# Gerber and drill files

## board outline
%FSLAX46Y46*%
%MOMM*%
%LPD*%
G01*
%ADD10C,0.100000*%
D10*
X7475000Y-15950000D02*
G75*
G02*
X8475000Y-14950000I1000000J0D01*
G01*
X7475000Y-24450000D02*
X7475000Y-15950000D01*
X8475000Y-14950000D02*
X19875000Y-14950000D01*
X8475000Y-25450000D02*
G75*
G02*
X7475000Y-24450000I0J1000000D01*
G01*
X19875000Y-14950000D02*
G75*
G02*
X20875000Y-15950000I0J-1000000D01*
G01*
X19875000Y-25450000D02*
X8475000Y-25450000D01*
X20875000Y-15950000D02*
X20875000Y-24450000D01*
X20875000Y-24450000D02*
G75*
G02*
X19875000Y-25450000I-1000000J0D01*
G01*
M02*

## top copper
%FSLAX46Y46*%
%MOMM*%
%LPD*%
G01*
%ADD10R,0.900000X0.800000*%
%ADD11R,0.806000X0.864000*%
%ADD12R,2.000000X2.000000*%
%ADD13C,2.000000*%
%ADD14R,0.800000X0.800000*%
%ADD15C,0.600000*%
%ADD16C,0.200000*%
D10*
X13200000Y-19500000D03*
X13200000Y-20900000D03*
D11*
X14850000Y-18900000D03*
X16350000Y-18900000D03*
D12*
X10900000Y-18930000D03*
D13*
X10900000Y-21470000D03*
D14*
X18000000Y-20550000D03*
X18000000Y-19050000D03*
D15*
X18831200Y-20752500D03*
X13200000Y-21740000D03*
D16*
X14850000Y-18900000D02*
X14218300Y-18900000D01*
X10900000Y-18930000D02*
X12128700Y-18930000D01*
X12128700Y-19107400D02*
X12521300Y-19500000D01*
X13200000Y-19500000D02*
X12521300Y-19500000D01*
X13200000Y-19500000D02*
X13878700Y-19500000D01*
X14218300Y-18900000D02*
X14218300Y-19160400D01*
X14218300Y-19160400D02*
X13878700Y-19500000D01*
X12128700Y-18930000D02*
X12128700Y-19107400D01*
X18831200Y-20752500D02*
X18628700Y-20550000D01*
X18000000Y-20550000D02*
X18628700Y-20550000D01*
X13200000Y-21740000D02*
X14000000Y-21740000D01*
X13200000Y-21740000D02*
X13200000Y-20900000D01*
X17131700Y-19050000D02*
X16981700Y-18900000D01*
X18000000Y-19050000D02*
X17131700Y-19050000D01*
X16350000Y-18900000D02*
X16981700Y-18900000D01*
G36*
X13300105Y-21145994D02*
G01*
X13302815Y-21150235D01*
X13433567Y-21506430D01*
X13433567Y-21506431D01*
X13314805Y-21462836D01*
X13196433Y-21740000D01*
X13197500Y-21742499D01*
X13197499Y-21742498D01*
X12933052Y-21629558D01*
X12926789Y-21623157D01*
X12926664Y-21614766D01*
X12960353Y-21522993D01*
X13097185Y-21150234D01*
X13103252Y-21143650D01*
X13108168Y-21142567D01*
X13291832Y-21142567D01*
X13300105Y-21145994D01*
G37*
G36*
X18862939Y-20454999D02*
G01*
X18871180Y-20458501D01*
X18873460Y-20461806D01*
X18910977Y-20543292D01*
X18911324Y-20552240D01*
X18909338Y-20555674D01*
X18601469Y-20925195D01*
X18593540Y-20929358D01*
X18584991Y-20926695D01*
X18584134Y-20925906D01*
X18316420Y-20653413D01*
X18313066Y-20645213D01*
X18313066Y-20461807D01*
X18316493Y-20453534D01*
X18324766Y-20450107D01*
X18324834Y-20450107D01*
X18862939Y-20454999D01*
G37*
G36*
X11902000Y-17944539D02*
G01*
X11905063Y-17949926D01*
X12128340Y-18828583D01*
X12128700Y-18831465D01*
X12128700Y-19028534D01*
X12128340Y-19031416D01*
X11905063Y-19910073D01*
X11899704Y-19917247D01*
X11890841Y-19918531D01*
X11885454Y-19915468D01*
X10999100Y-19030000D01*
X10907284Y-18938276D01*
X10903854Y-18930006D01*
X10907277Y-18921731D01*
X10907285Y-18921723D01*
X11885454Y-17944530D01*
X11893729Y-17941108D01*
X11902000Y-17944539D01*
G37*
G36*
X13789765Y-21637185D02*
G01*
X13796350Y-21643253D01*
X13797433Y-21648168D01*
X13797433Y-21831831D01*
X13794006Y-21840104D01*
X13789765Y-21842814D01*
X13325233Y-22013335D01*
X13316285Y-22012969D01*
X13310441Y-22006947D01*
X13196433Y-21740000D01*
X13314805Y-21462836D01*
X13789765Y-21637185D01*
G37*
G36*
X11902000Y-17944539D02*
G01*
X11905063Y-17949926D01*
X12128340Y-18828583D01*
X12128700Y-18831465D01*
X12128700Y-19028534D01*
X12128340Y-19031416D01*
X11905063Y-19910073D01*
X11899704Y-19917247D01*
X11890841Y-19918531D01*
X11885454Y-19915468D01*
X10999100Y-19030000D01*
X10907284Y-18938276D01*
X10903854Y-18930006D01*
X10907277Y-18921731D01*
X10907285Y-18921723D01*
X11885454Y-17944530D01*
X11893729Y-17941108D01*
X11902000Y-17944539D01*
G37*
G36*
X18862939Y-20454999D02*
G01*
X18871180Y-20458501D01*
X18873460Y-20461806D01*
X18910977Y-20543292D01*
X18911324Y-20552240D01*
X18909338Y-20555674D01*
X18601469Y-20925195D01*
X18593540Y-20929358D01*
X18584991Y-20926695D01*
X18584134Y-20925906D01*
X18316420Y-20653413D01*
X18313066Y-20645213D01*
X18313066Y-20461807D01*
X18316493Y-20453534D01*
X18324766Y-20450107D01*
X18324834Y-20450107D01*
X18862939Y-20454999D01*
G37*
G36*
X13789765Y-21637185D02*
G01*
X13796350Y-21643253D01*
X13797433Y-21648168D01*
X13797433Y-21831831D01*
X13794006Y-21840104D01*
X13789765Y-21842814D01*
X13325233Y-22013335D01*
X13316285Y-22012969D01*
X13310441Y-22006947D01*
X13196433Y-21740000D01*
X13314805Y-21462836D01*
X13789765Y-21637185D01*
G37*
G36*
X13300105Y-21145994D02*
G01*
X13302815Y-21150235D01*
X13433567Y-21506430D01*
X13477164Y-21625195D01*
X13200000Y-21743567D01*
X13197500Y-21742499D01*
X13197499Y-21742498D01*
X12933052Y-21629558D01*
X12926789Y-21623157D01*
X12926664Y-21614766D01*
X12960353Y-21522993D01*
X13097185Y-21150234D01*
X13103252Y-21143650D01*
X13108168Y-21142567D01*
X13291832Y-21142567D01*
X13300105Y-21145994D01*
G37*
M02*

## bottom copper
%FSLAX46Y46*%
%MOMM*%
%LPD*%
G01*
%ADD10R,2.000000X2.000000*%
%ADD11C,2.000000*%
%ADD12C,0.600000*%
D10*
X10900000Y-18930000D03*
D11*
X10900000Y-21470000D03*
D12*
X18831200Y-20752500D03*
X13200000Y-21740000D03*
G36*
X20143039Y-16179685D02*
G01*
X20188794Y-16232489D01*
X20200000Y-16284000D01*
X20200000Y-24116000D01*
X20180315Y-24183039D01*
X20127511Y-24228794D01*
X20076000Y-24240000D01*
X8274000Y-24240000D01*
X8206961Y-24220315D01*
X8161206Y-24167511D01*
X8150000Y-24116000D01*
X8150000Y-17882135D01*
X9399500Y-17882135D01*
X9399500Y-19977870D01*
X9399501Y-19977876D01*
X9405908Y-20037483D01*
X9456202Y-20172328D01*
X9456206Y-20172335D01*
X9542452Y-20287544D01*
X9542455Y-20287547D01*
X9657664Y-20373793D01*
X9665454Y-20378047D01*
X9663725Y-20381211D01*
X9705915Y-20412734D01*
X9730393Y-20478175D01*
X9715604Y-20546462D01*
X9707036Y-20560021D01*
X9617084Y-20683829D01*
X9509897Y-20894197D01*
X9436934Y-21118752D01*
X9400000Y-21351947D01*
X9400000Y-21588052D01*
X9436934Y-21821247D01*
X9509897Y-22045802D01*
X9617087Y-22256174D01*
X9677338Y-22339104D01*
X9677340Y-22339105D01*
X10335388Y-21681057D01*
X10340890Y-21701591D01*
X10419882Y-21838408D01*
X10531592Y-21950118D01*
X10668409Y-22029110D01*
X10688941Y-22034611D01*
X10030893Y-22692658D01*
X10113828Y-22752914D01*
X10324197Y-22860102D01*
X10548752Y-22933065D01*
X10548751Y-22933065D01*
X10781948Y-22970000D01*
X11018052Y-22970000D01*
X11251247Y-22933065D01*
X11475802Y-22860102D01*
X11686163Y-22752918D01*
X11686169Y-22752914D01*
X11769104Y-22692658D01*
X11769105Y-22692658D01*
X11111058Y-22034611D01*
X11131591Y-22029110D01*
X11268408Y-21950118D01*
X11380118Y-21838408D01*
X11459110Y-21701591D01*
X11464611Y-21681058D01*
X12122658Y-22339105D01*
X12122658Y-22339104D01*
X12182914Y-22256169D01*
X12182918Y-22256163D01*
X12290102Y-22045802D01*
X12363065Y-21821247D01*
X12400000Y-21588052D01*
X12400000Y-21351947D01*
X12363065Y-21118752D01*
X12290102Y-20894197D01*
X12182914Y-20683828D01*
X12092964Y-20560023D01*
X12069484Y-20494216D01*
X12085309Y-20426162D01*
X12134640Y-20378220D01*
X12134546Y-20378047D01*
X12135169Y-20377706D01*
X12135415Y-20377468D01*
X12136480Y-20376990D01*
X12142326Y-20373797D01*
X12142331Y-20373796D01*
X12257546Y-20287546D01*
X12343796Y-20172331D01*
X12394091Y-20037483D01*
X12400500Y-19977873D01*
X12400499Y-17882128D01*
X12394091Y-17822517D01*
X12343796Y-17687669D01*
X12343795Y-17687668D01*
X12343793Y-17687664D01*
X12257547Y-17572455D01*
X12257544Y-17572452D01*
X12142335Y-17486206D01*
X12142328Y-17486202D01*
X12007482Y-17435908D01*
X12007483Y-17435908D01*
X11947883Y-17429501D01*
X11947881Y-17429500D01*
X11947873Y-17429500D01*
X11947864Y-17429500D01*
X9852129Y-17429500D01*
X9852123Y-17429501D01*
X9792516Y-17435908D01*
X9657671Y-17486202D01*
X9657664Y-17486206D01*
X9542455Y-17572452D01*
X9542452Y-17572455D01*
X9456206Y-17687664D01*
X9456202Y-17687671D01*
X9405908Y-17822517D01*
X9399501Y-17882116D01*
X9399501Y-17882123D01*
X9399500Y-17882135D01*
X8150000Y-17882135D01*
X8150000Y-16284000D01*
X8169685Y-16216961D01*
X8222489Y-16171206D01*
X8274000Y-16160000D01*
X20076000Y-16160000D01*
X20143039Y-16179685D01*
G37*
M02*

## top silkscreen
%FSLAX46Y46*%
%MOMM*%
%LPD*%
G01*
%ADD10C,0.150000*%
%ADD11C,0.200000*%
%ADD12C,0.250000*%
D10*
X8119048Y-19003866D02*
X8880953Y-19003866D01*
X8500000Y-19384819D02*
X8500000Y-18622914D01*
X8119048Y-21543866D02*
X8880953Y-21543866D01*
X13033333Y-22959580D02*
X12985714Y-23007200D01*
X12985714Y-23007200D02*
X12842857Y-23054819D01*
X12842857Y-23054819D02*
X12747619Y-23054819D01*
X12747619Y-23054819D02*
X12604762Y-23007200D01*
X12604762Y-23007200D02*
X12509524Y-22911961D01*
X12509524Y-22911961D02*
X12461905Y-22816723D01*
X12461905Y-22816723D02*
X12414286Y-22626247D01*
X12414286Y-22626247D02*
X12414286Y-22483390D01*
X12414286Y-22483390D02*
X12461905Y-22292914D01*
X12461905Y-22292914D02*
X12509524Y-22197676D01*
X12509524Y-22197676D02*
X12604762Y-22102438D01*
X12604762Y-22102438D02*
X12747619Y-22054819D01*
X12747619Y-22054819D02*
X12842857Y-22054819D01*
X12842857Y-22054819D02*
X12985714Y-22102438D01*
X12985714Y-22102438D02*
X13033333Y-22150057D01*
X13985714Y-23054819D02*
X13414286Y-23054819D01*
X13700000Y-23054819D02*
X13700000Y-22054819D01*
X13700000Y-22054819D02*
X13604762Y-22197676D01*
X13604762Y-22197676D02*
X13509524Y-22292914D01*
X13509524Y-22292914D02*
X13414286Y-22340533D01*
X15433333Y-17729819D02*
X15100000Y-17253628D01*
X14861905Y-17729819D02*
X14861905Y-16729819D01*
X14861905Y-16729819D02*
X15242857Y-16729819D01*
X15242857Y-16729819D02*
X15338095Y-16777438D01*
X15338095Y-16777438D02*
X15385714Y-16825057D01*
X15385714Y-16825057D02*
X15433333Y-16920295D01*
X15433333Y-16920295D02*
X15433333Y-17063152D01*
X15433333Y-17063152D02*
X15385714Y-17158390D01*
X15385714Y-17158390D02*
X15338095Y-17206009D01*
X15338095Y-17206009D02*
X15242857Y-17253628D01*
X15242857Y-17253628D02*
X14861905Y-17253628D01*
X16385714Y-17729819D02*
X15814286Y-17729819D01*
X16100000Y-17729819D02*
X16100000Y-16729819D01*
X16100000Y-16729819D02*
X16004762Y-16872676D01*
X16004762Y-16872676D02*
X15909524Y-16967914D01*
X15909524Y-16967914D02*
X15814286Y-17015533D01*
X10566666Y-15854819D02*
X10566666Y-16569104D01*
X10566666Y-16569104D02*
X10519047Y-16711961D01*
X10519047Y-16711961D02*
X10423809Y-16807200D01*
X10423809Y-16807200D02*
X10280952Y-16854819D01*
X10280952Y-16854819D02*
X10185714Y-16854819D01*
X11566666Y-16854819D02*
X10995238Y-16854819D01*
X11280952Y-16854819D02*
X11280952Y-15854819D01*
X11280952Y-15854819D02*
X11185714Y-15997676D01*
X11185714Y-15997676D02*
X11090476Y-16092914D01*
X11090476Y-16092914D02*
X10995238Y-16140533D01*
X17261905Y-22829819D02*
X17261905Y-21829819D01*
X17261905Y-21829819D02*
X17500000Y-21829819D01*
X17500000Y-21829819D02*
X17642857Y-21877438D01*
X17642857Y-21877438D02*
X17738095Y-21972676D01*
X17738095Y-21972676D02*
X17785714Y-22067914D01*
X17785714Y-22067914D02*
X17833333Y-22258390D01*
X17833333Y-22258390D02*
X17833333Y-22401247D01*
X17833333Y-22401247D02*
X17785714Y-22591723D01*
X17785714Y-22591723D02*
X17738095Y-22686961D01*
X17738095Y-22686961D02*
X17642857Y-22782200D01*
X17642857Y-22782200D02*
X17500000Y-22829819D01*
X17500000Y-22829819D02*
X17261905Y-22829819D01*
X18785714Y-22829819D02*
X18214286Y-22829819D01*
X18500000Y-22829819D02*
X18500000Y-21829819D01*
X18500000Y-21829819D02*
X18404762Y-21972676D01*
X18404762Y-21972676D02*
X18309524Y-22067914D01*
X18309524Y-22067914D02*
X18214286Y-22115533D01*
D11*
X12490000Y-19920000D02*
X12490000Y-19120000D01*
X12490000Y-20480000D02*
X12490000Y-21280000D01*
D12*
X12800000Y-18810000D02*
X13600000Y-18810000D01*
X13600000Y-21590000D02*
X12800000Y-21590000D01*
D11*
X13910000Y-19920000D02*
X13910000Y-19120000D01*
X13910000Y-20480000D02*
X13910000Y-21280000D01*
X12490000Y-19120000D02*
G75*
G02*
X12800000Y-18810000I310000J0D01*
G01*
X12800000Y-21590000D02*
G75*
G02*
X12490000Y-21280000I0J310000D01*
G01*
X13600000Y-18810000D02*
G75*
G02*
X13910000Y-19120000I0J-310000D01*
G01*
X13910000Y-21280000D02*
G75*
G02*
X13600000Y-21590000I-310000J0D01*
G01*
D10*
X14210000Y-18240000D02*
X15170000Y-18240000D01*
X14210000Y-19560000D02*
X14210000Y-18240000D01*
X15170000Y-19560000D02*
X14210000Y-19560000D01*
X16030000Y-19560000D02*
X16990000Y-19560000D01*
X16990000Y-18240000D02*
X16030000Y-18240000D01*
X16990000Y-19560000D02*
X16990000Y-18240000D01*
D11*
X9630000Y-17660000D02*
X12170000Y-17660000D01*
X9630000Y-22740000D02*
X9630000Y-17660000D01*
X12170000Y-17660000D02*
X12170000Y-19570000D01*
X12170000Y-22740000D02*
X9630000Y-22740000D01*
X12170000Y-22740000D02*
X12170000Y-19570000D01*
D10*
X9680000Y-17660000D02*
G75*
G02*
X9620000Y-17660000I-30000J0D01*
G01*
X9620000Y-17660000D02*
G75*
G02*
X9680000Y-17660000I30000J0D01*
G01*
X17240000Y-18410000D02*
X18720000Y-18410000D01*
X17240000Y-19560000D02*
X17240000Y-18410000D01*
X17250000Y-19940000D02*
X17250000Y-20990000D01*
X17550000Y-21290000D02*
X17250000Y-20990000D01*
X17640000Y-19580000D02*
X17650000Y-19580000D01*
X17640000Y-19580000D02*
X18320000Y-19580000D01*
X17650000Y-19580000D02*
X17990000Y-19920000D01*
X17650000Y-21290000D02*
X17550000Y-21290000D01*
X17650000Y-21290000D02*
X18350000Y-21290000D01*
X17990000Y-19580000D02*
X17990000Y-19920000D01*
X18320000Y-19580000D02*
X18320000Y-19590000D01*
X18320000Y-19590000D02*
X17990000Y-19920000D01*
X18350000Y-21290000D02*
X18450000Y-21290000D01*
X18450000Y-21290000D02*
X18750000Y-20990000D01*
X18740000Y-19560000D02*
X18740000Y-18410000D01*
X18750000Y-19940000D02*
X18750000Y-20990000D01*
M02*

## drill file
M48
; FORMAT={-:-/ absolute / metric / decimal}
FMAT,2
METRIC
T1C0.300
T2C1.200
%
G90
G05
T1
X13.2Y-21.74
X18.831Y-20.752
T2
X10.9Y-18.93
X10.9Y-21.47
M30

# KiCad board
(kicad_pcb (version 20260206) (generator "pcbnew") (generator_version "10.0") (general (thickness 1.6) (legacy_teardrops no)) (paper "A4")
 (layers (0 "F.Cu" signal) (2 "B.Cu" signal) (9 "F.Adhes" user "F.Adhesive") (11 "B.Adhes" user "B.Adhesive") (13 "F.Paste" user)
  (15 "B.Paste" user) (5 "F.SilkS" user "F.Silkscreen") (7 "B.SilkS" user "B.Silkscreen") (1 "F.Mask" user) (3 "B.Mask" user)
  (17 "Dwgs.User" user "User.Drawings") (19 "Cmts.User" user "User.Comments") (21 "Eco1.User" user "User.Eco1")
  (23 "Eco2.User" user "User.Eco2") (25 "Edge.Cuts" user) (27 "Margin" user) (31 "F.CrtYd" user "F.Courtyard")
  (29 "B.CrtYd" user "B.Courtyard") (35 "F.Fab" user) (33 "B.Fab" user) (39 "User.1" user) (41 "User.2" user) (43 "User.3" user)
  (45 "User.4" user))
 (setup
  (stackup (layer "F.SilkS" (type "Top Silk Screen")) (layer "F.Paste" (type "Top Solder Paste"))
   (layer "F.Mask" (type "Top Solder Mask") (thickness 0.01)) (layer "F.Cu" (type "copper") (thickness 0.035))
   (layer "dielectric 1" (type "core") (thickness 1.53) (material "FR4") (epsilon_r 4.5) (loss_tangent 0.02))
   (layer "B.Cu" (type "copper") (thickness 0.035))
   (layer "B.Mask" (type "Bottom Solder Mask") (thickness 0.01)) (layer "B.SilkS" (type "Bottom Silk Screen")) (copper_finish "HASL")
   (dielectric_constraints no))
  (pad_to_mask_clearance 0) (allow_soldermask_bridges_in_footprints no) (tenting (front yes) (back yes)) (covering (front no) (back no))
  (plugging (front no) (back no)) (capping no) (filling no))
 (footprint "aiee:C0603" (layer "F.Cu") (at 13.2 20.2 -90)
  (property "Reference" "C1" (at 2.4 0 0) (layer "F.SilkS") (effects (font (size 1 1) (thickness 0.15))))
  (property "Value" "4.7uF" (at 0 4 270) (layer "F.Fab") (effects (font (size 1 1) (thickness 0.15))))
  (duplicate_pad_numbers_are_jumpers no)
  (fp_line (start -0.28 0.71) (end -1.08 0.71) (stroke (width 0.2) (type solid)) (layer "F.SilkS"))
  (fp_line (start 0.28 0.71) (end 1.08 0.71) (stroke (width 0.2) (type solid)) (layer "F.SilkS"))
  (fp_line (start -1.39 0.4) (end -1.39 -0.4) (stroke (width 0.25) (type solid)) (layer "F.SilkS"))
  (fp_line (start 1.39 -0.4) (end 1.39 0.4) (stroke (width 0.25) (type solid)) (layer "F.SilkS"))
  (fp_line (start -0.28 -0.71) (end -1.08 -0.71) (stroke (width 0.2) (type solid)) (layer "F.SilkS"))
  (fp_line (start 0.28 -0.71) (end 1.08 -0.71) (stroke (width 0.2) (type solid)) (layer "F.SilkS"))
  (fp_arc (start -1.08 0.71) (mid -1.299203 0.619203) (end -1.39 0.4) (stroke (width 0.2) (type solid)) (layer "F.SilkS"))
  (fp_arc (start 1.39 0.4) (mid 1.299203 0.619203) (end 1.08 0.71) (stroke (width 0.2) (type solid)) (layer "F.SilkS"))
  (fp_arc (start -1.39 -0.4) (mid -1.299203 -0.619203) (end -1.08 -0.71) (stroke (width 0.2) (type solid)) (layer "F.SilkS"))
  (fp_arc (start 1.08 -0.71) (mid 1.299203 -0.619203) (end 1.39 -0.4) (stroke (width 0.2) (type solid)) (layer "F.SilkS"))
  (pad "1" smd rect (at -0.7 0 270) (size 0.8 0.9) (layers "F.Cu" "F.Mask" "F.Paste") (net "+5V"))
  (pad "2" smd rect (at 0.7 0 270) (size 0.8 0.9) (layers "F.Cu" "F.Mask" "F.Paste") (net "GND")))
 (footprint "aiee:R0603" (layer "F.Cu") (at 15.6 18.9)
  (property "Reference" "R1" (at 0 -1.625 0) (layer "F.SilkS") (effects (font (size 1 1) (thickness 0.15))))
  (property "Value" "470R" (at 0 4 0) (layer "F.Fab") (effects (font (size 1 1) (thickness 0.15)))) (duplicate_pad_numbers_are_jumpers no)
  (fp_line (start -1.39 -0.66) (end -0.43 -0.66) (stroke (width 0.15) (type solid)) (layer "F.SilkS"))
  (fp_line (start -1.39 0.66) (end -1.39 -0.66) (stroke (width 0.15) (type solid)) (layer "F.SilkS"))
  (fp_line (start -0.43 0.66) (end -1.39 0.66) (stroke (width 0.15) (type solid)) (layer "F.SilkS"))
  (fp_line (start 0.43 0.66) (end 1.39 0.66) (stroke (width 0.15) (type solid)) (layer "F.SilkS"))
  (fp_line (start 1.39 -0.66) (end 0.43 -0.66) (stroke (width 0.15) (type solid)) (layer "F.SilkS"))
  (fp_line (start 1.39 0.66) (end 1.39 -0.66) (stroke (width 0.15) (type solid)) (layer "F.SilkS"))
  (pad "1" smd rect (at -0.75 0) (size 0.806 0.864) (layers "F.Cu" "F.Mask" "F.Paste") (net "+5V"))
  (pad "2" smd rect (at 0.75 0) (size 0.806 0.864) (layers "F.Cu" "F.Mask" "F.Paste") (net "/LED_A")))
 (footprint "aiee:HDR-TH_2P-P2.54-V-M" (layer "F.Cu") (at 10.9 20.2 -90)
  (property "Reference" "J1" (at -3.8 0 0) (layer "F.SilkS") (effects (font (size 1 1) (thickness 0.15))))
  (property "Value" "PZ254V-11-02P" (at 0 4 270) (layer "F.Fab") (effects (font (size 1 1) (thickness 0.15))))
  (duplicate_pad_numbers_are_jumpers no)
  (fp_line (start -2.54 1.27) (end -2.54 -1.27) (stroke (width 0.2) (type solid)) (layer "F.SilkS"))
  (fp_line (start 2.54 1.27) (end -2.54 1.27) (stroke (width 0.2) (type solid)) (layer "F.SilkS"))
  (fp_line (start -2.54 -1.27) (end -0.63 -1.27) (stroke (width 0.2) (type solid)) (layer "F.SilkS"))
  (fp_line (start 2.54 -1.27) (end 2.54 1.27) (stroke (width 0.2) (type solid)) (layer "F.SilkS"))
  (fp_line (start 2.54 -1.27) (end -0.63 -1.27) (stroke (width 0.2) (type solid)) (layer "F.SilkS"))
  (fp_circle (center -2.54 1.25) (end -2.51 1.25) (stroke (width 0.15) (type solid)) (fill no) (layer "F.SilkS"))
  (pad "1" thru_hole rect (at -1.27 0 270) (size 2 2) (drill 1.199998) (layers "*.Cu" "*.Mask") (remove_unused_layers no) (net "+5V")
   (teardrops (best_length_ratio 0.5) (max_length 1) (best_width_ratio 1) (max_width 2) (curved_edges no) (filter_ratio 0.9) (enabled yes)
    (allow_two_segments yes) (prefer_zone_connections yes)))
  (pad "2" thru_hole circle (at 1.27 0 270) (size 2 2) (drill 1.199998) (layers "*.Cu" "*.Mask") (remove_unused_layers no) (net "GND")))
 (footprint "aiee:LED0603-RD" (layer "F.Cu") (at 18 19.8 90)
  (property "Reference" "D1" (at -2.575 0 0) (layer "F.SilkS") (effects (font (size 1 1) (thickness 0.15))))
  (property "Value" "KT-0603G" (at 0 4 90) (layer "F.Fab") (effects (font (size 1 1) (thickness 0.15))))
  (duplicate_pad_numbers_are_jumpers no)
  (fp_line (start 1.39 -0.76) (end 1.39 0.72) (stroke (width 0.15) (type solid)) (layer "F.SilkS"))
  (fp_line (start 0.24 -0.76) (end 1.39 -0.76) (stroke (width 0.15) (type solid)) (layer "F.SilkS"))
  (fp_line (start -0.14 -0.75) (end -1.19 -0.75) (stroke (width 0.15) (type solid)) (layer "F.SilkS"))
  (fp_line (start -1.49 -0.45) (end -1.19 -0.75) (stroke (width 0.15) (type solid)) (layer "F.SilkS"))
  (fp_line (start 0.22 -0.36) (end 0.22 -0.35) (stroke (width 0.15) (type solid)) (layer "F.SilkS"))
  (fp_line (start 0.22 -0.36) (end 0.22 0.32) (stroke (width 0.15) (type solid)) (layer "F.SilkS"))
  (fp_line (start 0.22 -0.35) (end -0.12 -0.01) (stroke (width 0.15) (type solid)) (layer "F.SilkS"))
  (fp_line (start -1.49 -0.35) (end -1.49 -0.45) (stroke (width 0.15) (type solid)) (layer "F.SilkS"))
  (fp_line (start -1.49 -0.35) (end -1.49 0.35) (stroke (width 0.15) (type solid)) (layer "F.SilkS"))
  (fp_line (start 0.22 -0.01) (end -0.12 -0.01) (stroke (width 0.15) (type solid)) (layer "F.SilkS"))
  (fp_line (start 0.22 0.32) (end 0.21 0.32) (stroke (width 0.15) (type solid)) (layer "F.SilkS"))
  (fp_line (start 0.21 0.32) (end -0.12 -0.01) (stroke (width 0.15) (type solid)) (layer "F.SilkS"))
  (fp_line (start -1.49 0.35) (end -1.49 0.45) (stroke (width 0.15) (type solid)) (layer "F.SilkS"))
  (fp_line (start -1.49 0.45) (end -1.19 0.75) (stroke (width 0.15) (type solid)) (layer "F.SilkS"))
  (fp_line (start 0.24 0.74) (end 1.39 0.74) (stroke (width 0.15) (type solid)) (layer "F.SilkS"))
  (fp_line (start -0.14 0.75) (end -1.19 0.75) (stroke (width 0.15) (type solid)) (layer "F.SilkS"))
  (pad "1" smd rect (at -0.75 0 180) (size 0.8 0.8) (layers "F.Cu" "F.Mask" "F.Paste") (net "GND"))
  (pad "2" smd rect (at 0.75 0 180) (size 0.8 0.8) (layers "F.Cu" "F.Mask" "F.Paste") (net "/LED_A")))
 (gr_arc (start 7.475 15.95) (mid 7.767893 15.242893) (end 8.475 14.95) (stroke (width 0.1) (type default)) (layer "Edge.Cuts"))
 (gr_line (start 7.475 24.45) (end 7.475 15.95) (stroke (width 0.1) (type default)) (layer "Edge.Cuts"))
 (gr_line (start 8.475 14.95) (end 19.875 14.95) (stroke (width 0.1) (type default)) (layer "Edge.Cuts"))
 (gr_arc (start 8.475 25.45) (mid 7.767893 25.157106) (end 7.475 24.45) (stroke (width 0.1) (type default)) (layer "Edge.Cuts"))
 (gr_arc (start 19.875 14.95) (mid 20.582106 15.242893) (end 20.875 15.95) (stroke (width 0.1) (type default)) (layer "Edge.Cuts"))
 (gr_line (start 19.875 25.45) (end 8.475 25.45) (stroke (width 0.1) (type default)) (layer "Edge.Cuts"))
 (gr_line (start 20.875 15.95) (end 20.875 24.45) (stroke (width 0.1) (type default)) (layer "Edge.Cuts"))
 (gr_arc (start 20.875 24.45) (mid 20.582106 25.157106) (end 19.875 25.45) (stroke (width 0.1) (type default)) (layer "Edge.Cuts"))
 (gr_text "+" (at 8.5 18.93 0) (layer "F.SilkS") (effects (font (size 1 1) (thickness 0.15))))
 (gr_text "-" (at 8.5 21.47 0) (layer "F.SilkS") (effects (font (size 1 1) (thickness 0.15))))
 (segment (start 14.85 18.9) (end 14.2183 18.9) (width 0.2) (layer "F.Cu") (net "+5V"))
 (segment (start 10.9 18.93) (end 12.1287 18.93) (width 0.2) (layer "F.Cu") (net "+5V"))
 (segment (start 12.1287 19.1074) (end 12.5213 19.5) (width 0.2) (layer "F.Cu") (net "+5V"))
 (segment (start 13.2 19.5) (end 12.5213 19.5) (width 0.2) (layer "F.Cu") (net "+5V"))
 (segment (start 13.2 19.5) (end 13.8787 19.5) (width 0.2) (layer "F.Cu") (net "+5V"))
 (segment (start 14.2183 18.9) (end 14.2183 19.1604) (width 0.2) (layer "F.Cu") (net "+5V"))
 (segment (start 14.2183 19.1604) (end 13.8787 19.5) (width 0.2) (layer "F.Cu") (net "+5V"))
 (segment (start 12.1287 18.93) (end 12.1287 19.1074) (width 0.2) (layer "F.Cu") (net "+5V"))
 (segment (start 18.8312 20.7525) (end 18.6287 20.55) (width 0.2) (layer "F.Cu") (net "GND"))
 (segment (start 18 20.55) (end 18.6287 20.55) (width 0.2) (layer "F.Cu") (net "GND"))
 (segment (start 13.2 21.74) (end 14 21.74) (width 0.2) (layer "F.Cu") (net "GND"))
 (segment (start 13.2 21.74) (end 13.2 20.9) (width 0.2) (layer "F.Cu") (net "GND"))
 (via (at 18.8312 20.7525) (size 0.6) (drill 0.3) (layers "F.Cu" "B.Cu")
  (teardrops (best_length_ratio 0.5) (max_length 1) (best_width_ratio 1) (max_width 2) (curved_edges no) (filter_ratio 0.9) (enabled yes)
   (allow_two_segments yes) (prefer_zone_connections yes))
  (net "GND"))
 (via (at 13.2 21.74) (size 0.6) (drill 0.3) (layers "F.Cu" "B.Cu")
  (teardrops (best_length_ratio 0.5) (max_length 1) (best_width_ratio 1) (max_width 2) (curved_edges no) (filter_ratio 0.9) (enabled yes)
   (allow_two_segments yes) (prefer_zone_connections yes))
  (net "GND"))
 (segment (start 17.1317 19.05) (end 16.9817 18.9) (width 0.2) (layer "F.Cu") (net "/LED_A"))
 (segment (start 18 19.05) (end 17.1317 19.05) (width 0.2) (layer "F.Cu") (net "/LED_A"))
 (segment (start 16.35 18.9) (end 16.9817 18.9) (width 0.2) (layer "F.Cu") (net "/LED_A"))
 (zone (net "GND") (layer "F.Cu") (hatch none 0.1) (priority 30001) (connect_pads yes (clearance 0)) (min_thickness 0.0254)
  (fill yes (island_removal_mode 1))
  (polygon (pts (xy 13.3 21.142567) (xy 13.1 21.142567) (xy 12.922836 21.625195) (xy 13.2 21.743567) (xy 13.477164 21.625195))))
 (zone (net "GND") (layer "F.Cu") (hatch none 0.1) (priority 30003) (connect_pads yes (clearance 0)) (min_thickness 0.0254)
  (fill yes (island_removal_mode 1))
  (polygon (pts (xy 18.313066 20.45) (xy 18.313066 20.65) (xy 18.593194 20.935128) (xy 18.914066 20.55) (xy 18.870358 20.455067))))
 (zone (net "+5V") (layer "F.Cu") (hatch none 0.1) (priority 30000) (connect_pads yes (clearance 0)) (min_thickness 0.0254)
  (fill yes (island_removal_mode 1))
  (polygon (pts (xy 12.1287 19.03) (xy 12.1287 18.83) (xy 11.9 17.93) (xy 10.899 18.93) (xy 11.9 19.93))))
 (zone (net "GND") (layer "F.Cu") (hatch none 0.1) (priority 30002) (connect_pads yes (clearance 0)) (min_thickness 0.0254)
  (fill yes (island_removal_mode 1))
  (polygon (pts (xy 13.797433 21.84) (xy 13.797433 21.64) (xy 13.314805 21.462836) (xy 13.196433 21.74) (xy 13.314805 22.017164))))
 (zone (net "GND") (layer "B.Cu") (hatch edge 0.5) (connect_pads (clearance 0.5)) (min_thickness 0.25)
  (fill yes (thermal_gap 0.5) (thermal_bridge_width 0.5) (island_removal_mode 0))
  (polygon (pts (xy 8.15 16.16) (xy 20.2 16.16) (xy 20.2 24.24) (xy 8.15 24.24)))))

